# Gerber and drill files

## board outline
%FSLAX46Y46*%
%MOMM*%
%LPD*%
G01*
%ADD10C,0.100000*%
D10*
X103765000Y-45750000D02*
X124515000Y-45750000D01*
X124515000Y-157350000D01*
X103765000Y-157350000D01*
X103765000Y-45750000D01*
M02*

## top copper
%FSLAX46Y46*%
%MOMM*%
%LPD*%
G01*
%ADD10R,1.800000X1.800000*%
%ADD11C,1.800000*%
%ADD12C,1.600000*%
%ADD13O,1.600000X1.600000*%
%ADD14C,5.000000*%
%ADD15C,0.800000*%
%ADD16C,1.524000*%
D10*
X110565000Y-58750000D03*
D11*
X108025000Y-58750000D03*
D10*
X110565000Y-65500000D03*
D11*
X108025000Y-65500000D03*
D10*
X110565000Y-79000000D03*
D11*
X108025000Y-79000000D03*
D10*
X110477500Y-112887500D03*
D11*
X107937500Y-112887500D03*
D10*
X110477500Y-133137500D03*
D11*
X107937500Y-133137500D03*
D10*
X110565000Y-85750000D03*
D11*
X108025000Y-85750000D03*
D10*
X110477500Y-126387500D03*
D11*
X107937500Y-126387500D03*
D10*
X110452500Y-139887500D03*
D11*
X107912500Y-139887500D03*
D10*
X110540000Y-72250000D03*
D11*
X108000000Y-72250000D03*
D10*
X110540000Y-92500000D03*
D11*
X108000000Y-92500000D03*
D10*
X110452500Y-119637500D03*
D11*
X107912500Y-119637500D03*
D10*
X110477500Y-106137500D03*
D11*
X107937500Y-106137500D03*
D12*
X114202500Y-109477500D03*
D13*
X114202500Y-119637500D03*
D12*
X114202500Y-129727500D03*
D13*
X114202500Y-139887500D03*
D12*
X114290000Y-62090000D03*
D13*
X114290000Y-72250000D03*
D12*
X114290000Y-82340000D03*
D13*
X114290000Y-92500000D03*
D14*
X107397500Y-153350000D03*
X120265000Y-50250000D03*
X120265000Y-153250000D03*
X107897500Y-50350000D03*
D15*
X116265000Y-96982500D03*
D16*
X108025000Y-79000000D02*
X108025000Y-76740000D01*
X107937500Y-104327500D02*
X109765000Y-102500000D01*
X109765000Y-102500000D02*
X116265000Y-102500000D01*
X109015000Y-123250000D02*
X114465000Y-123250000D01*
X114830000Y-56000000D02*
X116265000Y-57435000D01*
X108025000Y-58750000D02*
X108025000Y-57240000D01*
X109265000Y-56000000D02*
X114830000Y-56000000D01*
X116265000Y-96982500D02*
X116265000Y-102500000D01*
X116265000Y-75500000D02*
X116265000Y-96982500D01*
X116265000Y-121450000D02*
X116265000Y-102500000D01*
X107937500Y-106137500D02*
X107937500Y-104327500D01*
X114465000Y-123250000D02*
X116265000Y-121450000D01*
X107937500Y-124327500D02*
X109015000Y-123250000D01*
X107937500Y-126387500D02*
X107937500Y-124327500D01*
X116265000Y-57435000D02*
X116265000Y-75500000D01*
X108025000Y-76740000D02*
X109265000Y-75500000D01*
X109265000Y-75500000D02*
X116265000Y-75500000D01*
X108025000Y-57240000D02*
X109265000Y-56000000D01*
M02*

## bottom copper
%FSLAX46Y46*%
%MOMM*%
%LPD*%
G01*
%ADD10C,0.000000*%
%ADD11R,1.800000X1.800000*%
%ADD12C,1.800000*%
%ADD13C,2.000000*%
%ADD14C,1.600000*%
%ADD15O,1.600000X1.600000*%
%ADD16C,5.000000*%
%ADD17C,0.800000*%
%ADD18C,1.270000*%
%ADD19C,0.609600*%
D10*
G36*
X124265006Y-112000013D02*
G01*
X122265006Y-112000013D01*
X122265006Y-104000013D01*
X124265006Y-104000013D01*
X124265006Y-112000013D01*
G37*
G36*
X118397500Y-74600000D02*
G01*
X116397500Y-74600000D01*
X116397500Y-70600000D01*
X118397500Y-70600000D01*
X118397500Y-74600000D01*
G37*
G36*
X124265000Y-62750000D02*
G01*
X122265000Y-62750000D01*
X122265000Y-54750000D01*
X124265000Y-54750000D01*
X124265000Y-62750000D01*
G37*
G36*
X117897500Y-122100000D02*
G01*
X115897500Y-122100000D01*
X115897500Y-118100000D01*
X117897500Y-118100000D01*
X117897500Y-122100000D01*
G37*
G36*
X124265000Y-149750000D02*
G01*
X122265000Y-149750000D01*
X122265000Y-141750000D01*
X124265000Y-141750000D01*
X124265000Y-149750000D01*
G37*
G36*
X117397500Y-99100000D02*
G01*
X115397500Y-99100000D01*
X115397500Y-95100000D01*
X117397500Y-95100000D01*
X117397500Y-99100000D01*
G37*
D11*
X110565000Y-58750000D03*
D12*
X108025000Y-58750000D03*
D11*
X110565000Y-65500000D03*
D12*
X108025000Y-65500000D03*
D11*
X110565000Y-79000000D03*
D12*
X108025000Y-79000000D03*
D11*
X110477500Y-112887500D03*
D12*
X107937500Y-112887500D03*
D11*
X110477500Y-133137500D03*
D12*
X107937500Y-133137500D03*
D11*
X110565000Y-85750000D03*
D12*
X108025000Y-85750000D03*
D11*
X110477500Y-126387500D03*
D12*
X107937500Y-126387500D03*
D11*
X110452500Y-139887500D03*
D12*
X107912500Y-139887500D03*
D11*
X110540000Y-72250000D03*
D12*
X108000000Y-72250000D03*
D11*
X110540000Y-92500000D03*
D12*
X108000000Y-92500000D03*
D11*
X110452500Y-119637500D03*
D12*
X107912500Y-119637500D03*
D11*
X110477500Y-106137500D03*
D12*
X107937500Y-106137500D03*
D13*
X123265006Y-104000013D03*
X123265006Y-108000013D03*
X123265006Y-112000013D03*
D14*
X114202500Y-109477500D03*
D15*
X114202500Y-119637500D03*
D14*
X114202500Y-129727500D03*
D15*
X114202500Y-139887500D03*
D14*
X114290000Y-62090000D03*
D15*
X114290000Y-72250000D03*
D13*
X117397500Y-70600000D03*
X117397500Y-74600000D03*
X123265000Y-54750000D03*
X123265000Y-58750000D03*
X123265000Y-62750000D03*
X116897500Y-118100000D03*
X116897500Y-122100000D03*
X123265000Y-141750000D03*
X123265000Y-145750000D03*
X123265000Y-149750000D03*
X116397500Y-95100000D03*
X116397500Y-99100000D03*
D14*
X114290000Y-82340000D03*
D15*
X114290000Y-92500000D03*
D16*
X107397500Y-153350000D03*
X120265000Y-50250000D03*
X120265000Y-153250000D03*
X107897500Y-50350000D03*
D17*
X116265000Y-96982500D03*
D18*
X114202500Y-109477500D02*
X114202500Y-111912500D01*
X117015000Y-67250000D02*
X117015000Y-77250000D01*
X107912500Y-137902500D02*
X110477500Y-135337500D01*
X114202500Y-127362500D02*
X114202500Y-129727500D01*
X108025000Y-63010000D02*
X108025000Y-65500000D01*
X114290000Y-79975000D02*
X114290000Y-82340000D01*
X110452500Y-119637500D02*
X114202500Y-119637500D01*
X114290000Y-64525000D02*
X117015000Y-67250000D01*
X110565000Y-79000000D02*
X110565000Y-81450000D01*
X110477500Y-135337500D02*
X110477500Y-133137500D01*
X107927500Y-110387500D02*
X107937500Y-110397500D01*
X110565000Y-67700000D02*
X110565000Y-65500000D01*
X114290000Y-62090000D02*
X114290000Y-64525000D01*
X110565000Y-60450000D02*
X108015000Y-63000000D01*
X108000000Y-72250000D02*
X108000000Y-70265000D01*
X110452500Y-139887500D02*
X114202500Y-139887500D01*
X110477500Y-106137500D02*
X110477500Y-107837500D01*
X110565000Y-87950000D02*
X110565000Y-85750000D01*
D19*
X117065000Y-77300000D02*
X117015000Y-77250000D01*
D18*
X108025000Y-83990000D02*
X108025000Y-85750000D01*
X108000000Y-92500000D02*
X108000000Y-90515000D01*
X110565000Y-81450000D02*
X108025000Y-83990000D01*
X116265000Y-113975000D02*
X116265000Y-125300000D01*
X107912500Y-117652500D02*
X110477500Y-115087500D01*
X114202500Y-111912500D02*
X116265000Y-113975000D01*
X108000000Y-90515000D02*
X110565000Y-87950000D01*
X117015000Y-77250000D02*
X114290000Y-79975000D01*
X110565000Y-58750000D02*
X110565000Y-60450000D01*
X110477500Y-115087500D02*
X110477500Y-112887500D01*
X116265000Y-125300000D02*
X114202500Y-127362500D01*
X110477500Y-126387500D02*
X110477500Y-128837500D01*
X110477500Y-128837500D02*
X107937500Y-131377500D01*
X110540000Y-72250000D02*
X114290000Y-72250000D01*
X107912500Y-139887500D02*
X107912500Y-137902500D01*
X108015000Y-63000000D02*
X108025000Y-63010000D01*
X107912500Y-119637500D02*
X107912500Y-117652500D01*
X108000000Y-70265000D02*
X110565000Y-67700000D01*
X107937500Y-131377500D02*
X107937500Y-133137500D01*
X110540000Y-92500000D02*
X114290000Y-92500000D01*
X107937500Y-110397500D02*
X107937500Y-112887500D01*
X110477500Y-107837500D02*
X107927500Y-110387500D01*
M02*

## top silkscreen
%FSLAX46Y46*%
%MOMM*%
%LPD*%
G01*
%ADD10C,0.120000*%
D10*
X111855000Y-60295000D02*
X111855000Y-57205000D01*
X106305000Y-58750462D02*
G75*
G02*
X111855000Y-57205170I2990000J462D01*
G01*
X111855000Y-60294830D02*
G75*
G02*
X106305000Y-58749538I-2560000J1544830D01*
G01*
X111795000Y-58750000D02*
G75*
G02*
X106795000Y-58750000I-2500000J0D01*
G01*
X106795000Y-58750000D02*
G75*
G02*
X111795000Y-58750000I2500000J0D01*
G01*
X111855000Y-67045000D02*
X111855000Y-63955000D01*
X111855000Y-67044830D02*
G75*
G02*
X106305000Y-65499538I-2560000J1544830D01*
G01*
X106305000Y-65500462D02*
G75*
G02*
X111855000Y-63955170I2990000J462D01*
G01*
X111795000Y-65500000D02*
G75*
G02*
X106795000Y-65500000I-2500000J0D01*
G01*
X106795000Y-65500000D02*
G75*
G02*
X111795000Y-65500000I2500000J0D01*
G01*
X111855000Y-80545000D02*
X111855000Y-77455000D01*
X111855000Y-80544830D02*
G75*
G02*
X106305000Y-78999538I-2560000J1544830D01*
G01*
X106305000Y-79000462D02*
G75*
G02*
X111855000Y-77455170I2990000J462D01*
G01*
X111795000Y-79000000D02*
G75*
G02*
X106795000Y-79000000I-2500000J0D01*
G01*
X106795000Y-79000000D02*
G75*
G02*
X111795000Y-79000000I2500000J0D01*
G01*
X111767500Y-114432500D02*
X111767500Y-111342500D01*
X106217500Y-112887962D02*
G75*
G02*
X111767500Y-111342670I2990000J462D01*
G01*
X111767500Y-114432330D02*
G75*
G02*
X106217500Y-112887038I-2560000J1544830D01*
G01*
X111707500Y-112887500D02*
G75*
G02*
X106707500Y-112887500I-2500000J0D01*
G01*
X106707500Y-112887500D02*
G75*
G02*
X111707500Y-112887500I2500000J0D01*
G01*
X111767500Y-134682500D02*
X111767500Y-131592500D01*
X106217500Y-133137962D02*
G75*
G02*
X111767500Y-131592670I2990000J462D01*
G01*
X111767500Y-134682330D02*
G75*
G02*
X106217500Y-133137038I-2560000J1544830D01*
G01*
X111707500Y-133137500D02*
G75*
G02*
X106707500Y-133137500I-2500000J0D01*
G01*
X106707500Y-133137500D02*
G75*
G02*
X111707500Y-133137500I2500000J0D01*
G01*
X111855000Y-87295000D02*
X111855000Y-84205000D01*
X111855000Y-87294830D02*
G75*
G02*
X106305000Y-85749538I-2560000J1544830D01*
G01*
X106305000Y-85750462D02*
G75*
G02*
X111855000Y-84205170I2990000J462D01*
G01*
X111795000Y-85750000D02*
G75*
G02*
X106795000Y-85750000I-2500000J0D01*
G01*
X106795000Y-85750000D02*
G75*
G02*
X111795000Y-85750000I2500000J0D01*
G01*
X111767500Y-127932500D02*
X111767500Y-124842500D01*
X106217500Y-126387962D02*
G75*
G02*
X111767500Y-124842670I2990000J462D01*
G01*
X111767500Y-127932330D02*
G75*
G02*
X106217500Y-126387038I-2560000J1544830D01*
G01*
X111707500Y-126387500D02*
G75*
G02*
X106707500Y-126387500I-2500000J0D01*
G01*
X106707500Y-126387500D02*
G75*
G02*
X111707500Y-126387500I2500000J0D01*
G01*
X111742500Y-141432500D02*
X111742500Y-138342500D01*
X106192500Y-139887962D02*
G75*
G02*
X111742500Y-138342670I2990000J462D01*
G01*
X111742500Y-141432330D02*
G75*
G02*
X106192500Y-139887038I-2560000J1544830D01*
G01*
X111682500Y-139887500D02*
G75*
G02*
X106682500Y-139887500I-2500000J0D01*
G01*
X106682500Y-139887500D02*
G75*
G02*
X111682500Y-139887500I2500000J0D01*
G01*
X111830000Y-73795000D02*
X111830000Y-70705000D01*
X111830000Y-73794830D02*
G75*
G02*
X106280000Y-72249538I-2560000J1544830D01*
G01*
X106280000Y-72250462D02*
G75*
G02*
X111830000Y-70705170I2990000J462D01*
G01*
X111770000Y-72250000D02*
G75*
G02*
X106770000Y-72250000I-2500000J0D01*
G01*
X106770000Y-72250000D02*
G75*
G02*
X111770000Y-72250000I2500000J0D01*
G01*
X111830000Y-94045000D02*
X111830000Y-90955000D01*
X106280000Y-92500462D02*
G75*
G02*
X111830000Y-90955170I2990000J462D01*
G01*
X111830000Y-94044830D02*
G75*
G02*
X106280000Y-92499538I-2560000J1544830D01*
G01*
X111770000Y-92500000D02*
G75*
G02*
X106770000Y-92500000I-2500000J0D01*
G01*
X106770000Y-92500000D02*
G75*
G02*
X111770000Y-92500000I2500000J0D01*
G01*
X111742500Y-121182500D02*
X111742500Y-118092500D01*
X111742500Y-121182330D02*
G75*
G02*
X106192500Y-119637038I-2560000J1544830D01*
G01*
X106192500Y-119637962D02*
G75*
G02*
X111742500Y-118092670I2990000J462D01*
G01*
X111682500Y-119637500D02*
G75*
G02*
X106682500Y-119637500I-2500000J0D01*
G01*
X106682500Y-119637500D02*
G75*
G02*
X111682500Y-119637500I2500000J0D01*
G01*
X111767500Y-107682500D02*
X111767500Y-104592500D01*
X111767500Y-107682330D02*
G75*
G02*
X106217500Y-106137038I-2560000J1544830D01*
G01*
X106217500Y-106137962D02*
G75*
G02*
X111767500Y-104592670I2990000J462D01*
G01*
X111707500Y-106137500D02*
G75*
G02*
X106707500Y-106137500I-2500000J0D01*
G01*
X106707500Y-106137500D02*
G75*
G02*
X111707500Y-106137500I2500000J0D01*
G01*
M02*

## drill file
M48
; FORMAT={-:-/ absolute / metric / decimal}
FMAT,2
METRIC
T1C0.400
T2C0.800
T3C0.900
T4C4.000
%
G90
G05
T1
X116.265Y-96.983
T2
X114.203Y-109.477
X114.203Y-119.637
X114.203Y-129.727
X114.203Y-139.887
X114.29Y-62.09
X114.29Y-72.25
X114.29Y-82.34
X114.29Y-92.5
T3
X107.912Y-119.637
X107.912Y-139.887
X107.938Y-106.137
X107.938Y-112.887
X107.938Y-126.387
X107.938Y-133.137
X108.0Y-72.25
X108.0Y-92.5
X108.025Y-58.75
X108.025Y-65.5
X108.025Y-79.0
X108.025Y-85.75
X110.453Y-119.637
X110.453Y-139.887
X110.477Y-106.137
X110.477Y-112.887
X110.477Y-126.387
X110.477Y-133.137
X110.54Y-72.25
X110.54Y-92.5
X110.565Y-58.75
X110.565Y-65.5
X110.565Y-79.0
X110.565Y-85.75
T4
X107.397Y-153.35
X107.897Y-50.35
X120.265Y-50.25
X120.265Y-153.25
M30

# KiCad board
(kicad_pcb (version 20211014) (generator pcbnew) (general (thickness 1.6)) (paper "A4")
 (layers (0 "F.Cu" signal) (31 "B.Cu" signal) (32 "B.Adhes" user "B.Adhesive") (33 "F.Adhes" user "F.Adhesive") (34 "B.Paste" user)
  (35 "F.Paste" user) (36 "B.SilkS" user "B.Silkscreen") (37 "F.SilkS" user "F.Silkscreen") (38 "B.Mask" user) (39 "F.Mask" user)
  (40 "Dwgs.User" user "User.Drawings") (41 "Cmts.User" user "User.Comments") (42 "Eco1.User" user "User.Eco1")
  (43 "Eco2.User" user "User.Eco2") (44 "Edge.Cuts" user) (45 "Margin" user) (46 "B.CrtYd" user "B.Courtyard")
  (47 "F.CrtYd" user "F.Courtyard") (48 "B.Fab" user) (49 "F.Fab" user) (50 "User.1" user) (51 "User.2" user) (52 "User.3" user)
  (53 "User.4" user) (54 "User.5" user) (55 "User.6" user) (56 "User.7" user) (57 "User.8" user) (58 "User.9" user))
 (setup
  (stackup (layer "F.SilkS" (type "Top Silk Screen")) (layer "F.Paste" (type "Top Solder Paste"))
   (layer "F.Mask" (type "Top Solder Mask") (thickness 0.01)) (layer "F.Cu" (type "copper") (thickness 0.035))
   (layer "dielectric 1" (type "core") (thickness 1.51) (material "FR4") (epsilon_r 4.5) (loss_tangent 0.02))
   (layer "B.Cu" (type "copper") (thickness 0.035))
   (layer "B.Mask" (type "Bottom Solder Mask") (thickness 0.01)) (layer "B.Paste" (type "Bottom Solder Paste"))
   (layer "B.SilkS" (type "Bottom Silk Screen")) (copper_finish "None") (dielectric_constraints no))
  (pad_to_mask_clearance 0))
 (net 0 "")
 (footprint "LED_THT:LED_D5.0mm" (layer "F.Cu") (at 110.565 58.75 180)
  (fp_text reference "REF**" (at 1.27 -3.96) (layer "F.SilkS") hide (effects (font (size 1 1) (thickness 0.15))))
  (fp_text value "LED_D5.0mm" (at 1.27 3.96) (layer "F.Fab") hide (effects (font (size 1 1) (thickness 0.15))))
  (fp_line (start -1.29 -1.545) (end -1.29 1.545) (layer "F.SilkS") (width 0.12))
  (fp_arc (start 4.26 -0.000462) (mid 2.072002 2.880433) (end -1.29 1.54483) (layer "F.SilkS") (width 0.12))
  (fp_arc (start -1.29 -1.54483) (mid 2.072002 -2.880433) (end 4.26 0.000462) (layer "F.SilkS") (width 0.12))
  (fp_circle (center 1.27 0) (end 3.77 0) (layer "F.SilkS") (width 0.12) (fill none))
  (pad "1" thru_hole rect (at 0 0 180) (size 1.8 1.8) (drill 0.9) (layers *.Cu *.Mask))
  (pad "2" thru_hole circle (at 2.54 0 180) (size 1.8 1.8) (drill 0.9) (layers *.Cu *.Mask)))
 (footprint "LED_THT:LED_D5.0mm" (layer "F.Cu") (at 110.565 65.5 180)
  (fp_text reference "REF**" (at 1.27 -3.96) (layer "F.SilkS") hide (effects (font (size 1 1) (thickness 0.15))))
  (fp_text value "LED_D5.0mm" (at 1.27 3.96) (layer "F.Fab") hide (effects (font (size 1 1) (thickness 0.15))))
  (fp_line (start -1.29 -1.545) (end -1.29 1.545) (layer "F.SilkS") (width 0.12))
  (fp_arc (start -1.29 -1.54483) (mid 2.072002 -2.880433) (end 4.26 0.000462) (layer "F.SilkS") (width 0.12))
  (fp_arc (start 4.26 -0.000462) (mid 2.072002 2.880433) (end -1.29 1.54483) (layer "F.SilkS") (width 0.12))
  (fp_circle (center 1.27 0) (end 3.77 0) (layer "F.SilkS") (width 0.12) (fill none))
  (pad "1" thru_hole rect (at 0 0 180) (size 1.8 1.8) (drill 0.9) (layers *.Cu *.Mask))
  (pad "2" thru_hole circle (at 2.54 0 180) (size 1.8 1.8) (drill 0.9) (layers *.Cu *.Mask)))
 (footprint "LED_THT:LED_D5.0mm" (layer "F.Cu") (at 110.565 79 180)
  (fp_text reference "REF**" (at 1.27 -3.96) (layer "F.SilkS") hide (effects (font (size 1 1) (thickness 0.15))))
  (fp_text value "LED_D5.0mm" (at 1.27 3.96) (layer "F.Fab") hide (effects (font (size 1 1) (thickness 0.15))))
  (fp_line (start -1.29 -1.545) (end -1.29 1.545) (layer "F.SilkS") (width 0.12))
  (fp_arc (start -1.29 -1.54483) (mid 2.072002 -2.880433) (end 4.26 0.000462) (layer "F.SilkS") (width 0.12))
  (fp_arc (start 4.26 -0.000462) (mid 2.072002 2.880433) (end -1.29 1.54483) (layer "F.SilkS") (width 0.12))
  (fp_circle (center 1.27 0) (end 3.77 0) (layer "F.SilkS") (width 0.12) (fill none))
  (pad "1" thru_hole rect (at 0 0 180) (size 1.8 1.8) (drill 0.9) (layers *.Cu *.Mask))
  (pad "2" thru_hole circle (at 2.54 0 180) (size 1.8 1.8) (drill 0.9) (layers *.Cu *.Mask)))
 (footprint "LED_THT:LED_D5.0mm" (layer "F.Cu") (at 110.4775 112.8875 180)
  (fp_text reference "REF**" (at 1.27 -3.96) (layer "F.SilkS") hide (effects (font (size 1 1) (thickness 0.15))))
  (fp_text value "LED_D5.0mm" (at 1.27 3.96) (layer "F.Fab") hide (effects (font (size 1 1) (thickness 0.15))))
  (fp_line (start -1.29 -1.545) (end -1.29 1.545) (layer "F.SilkS") (width 0.12))
  (fp_arc (start 4.26 -0.000462) (mid 2.072002 2.880433) (end -1.29 1.54483) (layer "F.SilkS") (width 0.12))
  (fp_arc (start -1.29 -1.54483) (mid 2.072002 -2.880433) (end 4.26 0.000462) (layer "F.SilkS") (width 0.12))
  (fp_circle (center 1.27 0) (end 3.77 0) (layer "F.SilkS") (width 0.12) (fill none))
  (pad "1" thru_hole rect (at 0 0 180) (size 1.8 1.8) (drill 0.9) (layers *.Cu *.Mask))
  (pad "2" thru_hole circle (at 2.54 0 180) (size 1.8 1.8) (drill 0.9) (layers *.Cu *.Mask)))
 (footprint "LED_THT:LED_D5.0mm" (layer "F.Cu") (at 110.4775 133.1375 180)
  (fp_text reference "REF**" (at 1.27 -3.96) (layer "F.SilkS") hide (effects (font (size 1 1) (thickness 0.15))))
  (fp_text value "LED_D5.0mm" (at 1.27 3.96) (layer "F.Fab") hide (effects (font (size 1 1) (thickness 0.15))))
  (fp_line (start -1.29 -1.545) (end -1.29 1.545) (layer "F.SilkS") (width 0.12))
  (fp_arc (start 4.26 -0.000462) (mid 2.072002 2.880433) (end -1.29 1.54483) (layer "F.SilkS") (width 0.12))
  (fp_arc (start -1.29 -1.54483) (mid 2.072002 -2.880433) (end 4.26 0.000462) (layer "F.SilkS") (width 0.12))
  (fp_circle (center 1.27 0) (end 3.77 0) (layer "F.SilkS") (width 0.12) (fill none))
  (pad "1" thru_hole rect (at 0 0 180) (size 1.8 1.8) (drill 0.9) (layers *.Cu *.Mask))
  (pad "2" thru_hole circle (at 2.54 0 180) (size 1.8 1.8) (drill 0.9) (layers *.Cu *.Mask)))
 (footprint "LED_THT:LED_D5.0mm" (layer "F.Cu") (at 110.565 85.75 180)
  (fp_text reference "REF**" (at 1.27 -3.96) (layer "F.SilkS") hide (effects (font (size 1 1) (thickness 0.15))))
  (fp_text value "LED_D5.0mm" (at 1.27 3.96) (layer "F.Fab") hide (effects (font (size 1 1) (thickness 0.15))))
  (fp_line (start -1.29 -1.545) (end -1.29 1.545) (layer "F.SilkS") (width 0.12))
  (fp_arc (start -1.29 -1.54483) (mid 2.072002 -2.880433) (end 4.26 0.000462) (layer "F.SilkS") (width 0.12))
  (fp_arc (start 4.26 -0.000462) (mid 2.072002 2.880433) (end -1.29 1.54483) (layer "F.SilkS") (width 0.12))
  (fp_circle (center 1.27 0) (end 3.77 0) (layer "F.SilkS") (width 0.12) (fill none))
  (pad "1" thru_hole rect (at 0 0 180) (size 1.8 1.8) (drill 0.9) (layers *.Cu *.Mask))
  (pad "2" thru_hole circle (at 2.54 0 180) (size 1.8 1.8) (drill 0.9) (layers *.Cu *.Mask)))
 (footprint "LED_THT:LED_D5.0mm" (layer "F.Cu") (at 110.4775 126.3875 180)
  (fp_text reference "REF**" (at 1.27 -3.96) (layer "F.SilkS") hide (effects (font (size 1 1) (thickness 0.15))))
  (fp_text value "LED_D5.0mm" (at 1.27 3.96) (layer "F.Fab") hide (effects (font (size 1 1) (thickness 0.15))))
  (fp_line (start -1.29 -1.545) (end -1.29 1.545) (layer "F.SilkS") (width 0.12))
  (fp_arc (start 4.26 -0.000462) (mid 2.072002 2.880433) (end -1.29 1.54483) (layer "F.SilkS") (width 0.12))
  (fp_arc (start -1.29 -1.54483) (mid 2.072002 -2.880433) (end 4.26 0.000462) (layer "F.SilkS") (width 0.12))
  (fp_circle (center 1.27 0) (end 3.77 0) (layer "F.SilkS") (width 0.12) (fill none))
  (pad "1" thru_hole rect (at 0 0 180) (size 1.8 1.8) (drill 0.9) (layers *.Cu *.Mask))
  (pad "2" thru_hole circle (at 2.54 0 180) (size 1.8 1.8) (drill 0.9) (layers *.Cu *.Mask)))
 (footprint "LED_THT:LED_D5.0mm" (layer "F.Cu") (at 110.4525 139.8875 180)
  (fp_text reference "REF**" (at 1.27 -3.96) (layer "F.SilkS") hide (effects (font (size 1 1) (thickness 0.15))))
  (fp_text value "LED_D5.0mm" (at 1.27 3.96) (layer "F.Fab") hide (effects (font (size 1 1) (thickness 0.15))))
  (fp_line (start -1.29 -1.545) (end -1.29 1.545) (layer "F.SilkS") (width 0.12))
  (fp_arc (start 4.26 -0.000462) (mid 2.072002 2.880433) (end -1.29 1.54483) (layer "F.SilkS") (width 0.12))
  (fp_arc (start -1.29 -1.54483) (mid 2.072002 -2.880433) (end 4.26 0.000462) (layer "F.SilkS") (width 0.12))
  (fp_circle (center 1.27 0) (end 3.77 0) (layer "F.SilkS") (width 0.12) (fill none))
  (pad "1" thru_hole rect (at 0 0 180) (size 1.8 1.8) (drill 0.9) (layers *.Cu *.Mask))
  (pad "2" thru_hole circle (at 2.54 0 180) (size 1.8 1.8) (drill 0.9) (layers *.Cu *.Mask)))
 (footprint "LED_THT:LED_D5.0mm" (layer "F.Cu") (at 110.54 72.25 180)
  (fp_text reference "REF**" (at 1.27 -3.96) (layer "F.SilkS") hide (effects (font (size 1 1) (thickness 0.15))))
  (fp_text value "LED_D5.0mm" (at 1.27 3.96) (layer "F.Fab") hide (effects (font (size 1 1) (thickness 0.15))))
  (fp_line (start -1.29 -1.545) (end -1.29 1.545) (layer "F.SilkS") (width 0.12))
  (fp_arc (start -1.29 -1.54483) (mid 2.072002 -2.880433) (end 4.26 0.000462) (layer "F.SilkS") (width 0.12))
  (fp_arc (start 4.26 -0.000462) (mid 2.072002 2.880433) (end -1.29 1.54483) (layer "F.SilkS") (width 0.12))
  (fp_circle (center 1.27 0) (end 3.77 0) (layer "F.SilkS") (width 0.12) (fill none))
  (pad "1" thru_hole rect (at 0 0 180) (size 1.8 1.8) (drill 0.9) (layers *.Cu *.Mask))
  (pad "2" thru_hole circle (at 2.54 0 180) (size 1.8 1.8) (drill 0.9) (layers *.Cu *.Mask)))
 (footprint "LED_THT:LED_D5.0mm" (layer "F.Cu") (at 110.54 92.5 180)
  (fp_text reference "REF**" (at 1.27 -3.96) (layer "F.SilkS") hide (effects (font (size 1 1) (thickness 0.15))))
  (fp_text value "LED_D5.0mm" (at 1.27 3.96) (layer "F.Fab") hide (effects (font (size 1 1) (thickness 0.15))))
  (fp_line (start -1.29 -1.545) (end -1.29 1.545) (layer "F.SilkS") (width 0.12))
  (fp_arc (start 4.26 -0.000462) (mid 2.072002 2.880433) (end -1.29 1.54483) (layer "F.SilkS") (width 0.12))
  (fp_arc (start -1.29 -1.54483) (mid 2.072002 -2.880433) (end 4.26 0.000462) (layer "F.SilkS") (width 0.12))
  (fp_circle (center 1.27 0) (end 3.77 0) (layer "F.SilkS") (width 0.12) (fill none))
  (pad "1" thru_hole rect (at 0 0 180) (size 1.8 1.8) (drill 0.9) (layers *.Cu *.Mask))
  (pad "2" thru_hole circle (at 2.54 0 180) (size 1.8 1.8) (drill 0.9) (layers *.Cu *.Mask)))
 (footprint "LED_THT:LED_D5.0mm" (layer "F.Cu") (at 110.4525 119.6375 180)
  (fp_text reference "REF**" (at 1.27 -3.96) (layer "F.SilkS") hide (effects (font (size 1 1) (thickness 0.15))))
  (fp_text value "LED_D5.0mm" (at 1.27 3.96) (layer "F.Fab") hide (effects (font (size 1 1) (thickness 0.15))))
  (fp_line (start -1.29 -1.545) (end -1.29 1.545) (layer "F.SilkS") (width 0.12))
  (fp_arc (start -1.29 -1.54483) (mid 2.072002 -2.880433) (end 4.26 0.000462) (layer "F.SilkS") (width 0.12))
  (fp_arc (start 4.26 -0.000462) (mid 2.072002 2.880433) (end -1.29 1.54483) (layer "F.SilkS") (width 0.12))
  (fp_circle (center 1.27 0) (end 3.77 0) (layer "F.SilkS") (width 0.12) (fill none))
  (pad "1" thru_hole rect (at 0 0 180) (size 1.8 1.8) (drill 0.9) (layers *.Cu *.Mask))
  (pad "2" thru_hole circle (at 2.54 0 180) (size 1.8 1.8) (drill 0.9) (layers *.Cu *.Mask)))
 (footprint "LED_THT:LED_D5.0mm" (layer "F.Cu") (at 110.4775 106.1375 180)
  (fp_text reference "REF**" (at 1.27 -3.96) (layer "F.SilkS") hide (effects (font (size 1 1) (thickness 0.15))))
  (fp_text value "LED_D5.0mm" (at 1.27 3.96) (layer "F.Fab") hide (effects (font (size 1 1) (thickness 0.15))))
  (fp_line (start -1.29 -1.545) (end -1.29 1.545) (layer "F.SilkS") (width 0.12))
  (fp_arc (start -1.29 -1.54483) (mid 2.072002 -2.880433) (end 4.26 0.000462) (layer "F.SilkS") (width 0.12))
  (fp_arc (start 4.26 -0.000462) (mid 2.072002 2.880433) (end -1.29 1.54483) (layer "F.SilkS") (width 0.12))
  (fp_circle (center 1.27 0) (end 3.77 0) (layer "F.SilkS") (width 0.12) (fill none))
  (pad "1" thru_hole rect (at 0 0 180) (size 1.8 1.8) (drill 0.9) (layers *.Cu *.Mask))
  (pad "2" thru_hole circle (at 2.54 0 180) (size 1.8 1.8) (drill 0.9) (layers *.Cu *.Mask)))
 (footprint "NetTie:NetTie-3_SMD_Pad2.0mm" (layer "B.Cu") (at 123.265006 108.000013 -90)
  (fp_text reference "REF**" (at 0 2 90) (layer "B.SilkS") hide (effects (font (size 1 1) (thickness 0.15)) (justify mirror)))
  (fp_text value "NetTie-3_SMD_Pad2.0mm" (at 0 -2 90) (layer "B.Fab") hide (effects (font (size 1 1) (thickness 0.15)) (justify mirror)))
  (fp_poly (pts (xy -4 1) (xy 4 1) (xy 4 -1) (xy -4 -1)) (layer "B.Cu") (width 0) (fill solid))
  (pad "1" smd circle (at -4 0 270) (size 2 2) (layers "B.Cu")) (pad "2" smd circle (at 0 0 270) (size 2 2) (layers "B.Cu"))
  (pad "3" smd circle (at 4 0 270) (size 2 2) (layers "B.Cu")))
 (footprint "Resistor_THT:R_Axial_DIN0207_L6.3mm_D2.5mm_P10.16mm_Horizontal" (layer "B.Cu") (at 114.2025 109.4775 -90)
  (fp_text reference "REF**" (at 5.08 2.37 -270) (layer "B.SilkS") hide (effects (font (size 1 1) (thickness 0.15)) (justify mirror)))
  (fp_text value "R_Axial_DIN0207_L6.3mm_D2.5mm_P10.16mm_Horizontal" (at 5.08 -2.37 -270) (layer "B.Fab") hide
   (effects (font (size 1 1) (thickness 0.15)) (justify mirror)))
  (pad "1" thru_hole circle (at 0 0 270) (size 1.6 1.6) (drill 0.8) (layers *.Cu *.Mask))
  (pad "2" thru_hole oval (at 10.16 0 270) (size 1.6 1.6) (drill 0.8) (layers *.Cu *.Mask)))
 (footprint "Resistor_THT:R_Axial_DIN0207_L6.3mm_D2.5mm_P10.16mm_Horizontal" (layer "B.Cu") (at 114.2025 129.7275 -90)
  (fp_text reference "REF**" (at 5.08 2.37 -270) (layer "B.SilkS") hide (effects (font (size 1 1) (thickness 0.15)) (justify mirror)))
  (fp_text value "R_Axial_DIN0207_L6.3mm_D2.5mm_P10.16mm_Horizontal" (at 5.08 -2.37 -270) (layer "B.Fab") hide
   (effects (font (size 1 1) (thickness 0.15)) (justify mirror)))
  (pad "1" thru_hole circle (at 0 0 270) (size 1.6 1.6) (drill 0.8) (layers *.Cu *.Mask))
  (pad "2" thru_hole oval (at 10.16 0 270) (size 1.6 1.6) (drill 0.8) (layers *.Cu *.Mask)))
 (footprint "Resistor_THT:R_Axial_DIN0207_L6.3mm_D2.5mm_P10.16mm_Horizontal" (layer "B.Cu") (at 114.29 62.09 -90)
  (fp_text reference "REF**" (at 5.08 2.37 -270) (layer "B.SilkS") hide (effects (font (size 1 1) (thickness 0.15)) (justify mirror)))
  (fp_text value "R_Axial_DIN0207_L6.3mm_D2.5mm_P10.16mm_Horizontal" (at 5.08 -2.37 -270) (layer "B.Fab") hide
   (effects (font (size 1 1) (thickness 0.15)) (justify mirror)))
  (pad "1" thru_hole circle (at 0 0 270) (size 1.6 1.6) (drill 0.8) (layers *.Cu *.Mask))
  (pad "2" thru_hole oval (at 10.16 0 270) (size 1.6 1.6) (drill 0.8) (layers *.Cu *.Mask)))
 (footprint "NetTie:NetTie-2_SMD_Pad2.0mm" (layer "B.Cu") (at 117.3975 72.6 -90)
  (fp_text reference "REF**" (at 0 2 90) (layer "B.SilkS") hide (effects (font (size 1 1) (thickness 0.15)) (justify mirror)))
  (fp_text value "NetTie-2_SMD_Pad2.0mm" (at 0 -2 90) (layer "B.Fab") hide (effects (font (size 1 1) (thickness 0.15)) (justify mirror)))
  (fp_poly (pts (xy -2 1) (xy 2 1) (xy 2 -1) (xy -2 -1)) (layer "B.Cu") (width 0) (fill solid))
  (pad "1" smd circle (at -2 0 270) (size 2 2) (layers "B.Cu")) (pad "2" smd circle (at 2 0 270) (size 2 2) (layers "B.Cu")))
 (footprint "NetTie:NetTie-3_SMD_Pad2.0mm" (layer "B.Cu") (at 123.265 58.75 -90)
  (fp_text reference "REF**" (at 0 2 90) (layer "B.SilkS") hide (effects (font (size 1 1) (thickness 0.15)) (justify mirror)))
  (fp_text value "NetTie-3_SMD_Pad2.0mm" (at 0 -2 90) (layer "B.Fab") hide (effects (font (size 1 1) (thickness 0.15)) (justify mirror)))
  (fp_poly (pts (xy -4 1) (xy 4 1) (xy 4 -1) (xy -4 -1)) (layer "B.Cu") (width 0) (fill solid))
  (pad "1" smd circle (at -4 0 270) (size 2 2) (layers "B.Cu")) (pad "2" smd circle (at 0 0 270) (size 2 2) (layers "B.Cu"))
  (pad "3" smd circle (at 4 0 270) (size 2 2) (layers "B.Cu")))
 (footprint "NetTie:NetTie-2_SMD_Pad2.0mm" (layer "B.Cu") (at 116.8975 120.1 -90)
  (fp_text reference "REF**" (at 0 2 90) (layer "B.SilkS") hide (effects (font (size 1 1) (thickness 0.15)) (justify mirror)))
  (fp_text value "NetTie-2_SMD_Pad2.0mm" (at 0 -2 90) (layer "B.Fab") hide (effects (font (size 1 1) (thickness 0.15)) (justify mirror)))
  (fp_poly (pts (xy -2 1) (xy 2 1) (xy 2 -1) (xy -2 -1)) (layer "B.Cu") (width 0) (fill solid))
  (pad "1" smd circle (at -2 0 270) (size 2 2) (layers "B.Cu")) (pad "2" smd circle (at 2 0 270) (size 2 2) (layers "B.Cu")))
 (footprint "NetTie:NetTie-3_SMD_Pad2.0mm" (layer "B.Cu") (at 123.265 145.75 -90)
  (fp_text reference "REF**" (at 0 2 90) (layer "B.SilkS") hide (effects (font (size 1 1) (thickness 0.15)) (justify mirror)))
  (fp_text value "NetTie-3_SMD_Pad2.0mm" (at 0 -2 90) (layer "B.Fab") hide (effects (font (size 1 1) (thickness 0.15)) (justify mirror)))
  (fp_poly (pts (xy -4 1) (xy 4 1) (xy 4 -1) (xy -4 -1)) (layer "B.Cu") (width 0) (fill solid))
  (pad "1" smd circle (at -4 0 270) (size 2 2) (layers "B.Cu")) (pad "2" smd circle (at 0 0 270) (size 2 2) (layers "B.Cu"))
  (pad "3" smd circle (at 4 0 270) (size 2 2) (layers "B.Cu")))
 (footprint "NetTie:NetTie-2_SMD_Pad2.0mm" (layer "B.Cu") (at 116.3975 97.1 -90)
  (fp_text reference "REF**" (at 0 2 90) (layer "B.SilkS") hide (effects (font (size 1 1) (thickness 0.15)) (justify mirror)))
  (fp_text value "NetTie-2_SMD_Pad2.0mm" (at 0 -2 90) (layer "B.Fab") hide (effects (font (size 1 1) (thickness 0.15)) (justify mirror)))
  (fp_poly (pts (xy -2 1) (xy 2 1) (xy 2 -1) (xy -2 -1)) (layer "B.Cu") (width 0) (fill solid))
  (pad "1" smd circle (at -2 0 270) (size 2 2) (layers "B.Cu")) (pad "2" smd circle (at 2 0 270) (size 2 2) (layers "B.Cu")))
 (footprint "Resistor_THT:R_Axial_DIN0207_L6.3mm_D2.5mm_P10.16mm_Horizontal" (layer "B.Cu") (at 114.29 82.34 -90)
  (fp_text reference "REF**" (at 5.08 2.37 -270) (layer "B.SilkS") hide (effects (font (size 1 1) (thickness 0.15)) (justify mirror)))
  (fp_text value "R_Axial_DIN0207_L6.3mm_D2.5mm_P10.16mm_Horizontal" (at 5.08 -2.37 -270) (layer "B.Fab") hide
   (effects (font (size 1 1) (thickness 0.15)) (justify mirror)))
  (pad "1" thru_hole circle (at 0 0 270) (size 1.6 1.6) (drill 0.8) (layers *.Cu *.Mask))
  (pad "2" thru_hole oval (at 10.16 0 270) (size 1.6 1.6) (drill 0.8) (layers *.Cu *.Mask)))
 (gr_rect (start 124.515 157.35) (end 103.765 45.75) (layer "Edge.Cuts") (width 0.1) (fill none))
 (segment (start 108.025 79) (end 108.025 76.74) (width 1.524) (layer "F.Cu") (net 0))
 (segment (start 107.9375 104.3275) (end 109.765 102.5) (width 1.524) (layer "F.Cu") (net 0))
 (segment (start 109.765 102.5) (end 116.265 102.5) (width 1.524) (layer "F.Cu") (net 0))
 (segment (start 109.015 123.25) (end 114.465 123.25) (width 1.524) (layer "F.Cu") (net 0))
 (segment (start 114.83 56) (end 116.265 57.435) (width 1.524) (layer "F.Cu") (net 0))
 (segment (start 108.025 58.75) (end 108.025 57.24) (width 1.524) (layer "F.Cu") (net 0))
 (segment (start 109.265 56) (end 114.83 56) (width 1.524) (layer "F.Cu") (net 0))
 (segment (start 116.265 96.9825) (end 116.265 102.5) (width 1.524) (layer "F.Cu") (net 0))
 (segment (start 116.265 75.5) (end 116.265 96.9825) (width 1.524) (layer "F.Cu") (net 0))
 (segment (start 116.265 121.45) (end 116.265 102.5) (width 1.524) (layer "F.Cu") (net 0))
 (segment (start 107.9375 106.1375) (end 107.9375 104.3275) (width 1.524) (layer "F.Cu") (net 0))
 (segment (start 114.465 123.25) (end 116.265 121.45) (width 1.524) (layer "F.Cu") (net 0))
 (segment (start 107.9375 124.3275) (end 109.015 123.25) (width 1.524) (layer "F.Cu") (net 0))
 (segment (start 107.9375 126.3875) (end 107.9375 124.3275) (width 1.524) (layer "F.Cu") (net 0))
 (segment (start 116.265 57.435) (end 116.265 75.5) (width 1.524) (layer "F.Cu") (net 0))
 (segment (start 108.025 76.74) (end 109.265 75.5) (width 1.524) (layer "F.Cu") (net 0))
 (segment (start 109.265 75.5) (end 116.265 75.5) (width 1.524) (layer "F.Cu") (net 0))
 (segment (start 108.025 57.24) (end 109.265 56) (width 1.524) (layer "F.Cu") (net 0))
 (via (at 107.3975 153.35) (size 5) (drill 4) (layers "F.Cu" "B.Cu") (free) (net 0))
 (via (at 120.265 50.25) (size 5) (drill 4) (layers "F.Cu" "B.Cu") (free) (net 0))
 (via (at 120.265 153.25) (size 5) (drill 4) (layers "F.Cu" "B.Cu") (free) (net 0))
 (via (at 107.8975 50.35) (size 5) (drill 4) (layers "F.Cu" "B.Cu") (free) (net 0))
 (via (at 116.265 96.9825) (size 0.8) (drill 0.4) (layers "F.Cu" "B.Cu") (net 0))
 (segment (start 114.2025 109.4775) (end 114.2025 111.9125) (width 1.27) (layer "B.Cu") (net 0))
 (segment (start 117.015 67.25) (end 117.015 77.25) (width 1.27) (layer "B.Cu") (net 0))
 (segment (start 107.9125 137.9025) (end 110.4775 135.3375) (width 1.27) (layer "B.Cu") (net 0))
 (segment (start 114.2025 127.3625) (end 114.2025 129.7275) (width 1.27) (layer "B.Cu") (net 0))
 (segment (start 108.025 63.01) (end 108.025 65.5) (width 1.27) (layer "B.Cu") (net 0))
 (segment (start 114.29 79.975) (end 114.29 82.34) (width 1.27) (layer "B.Cu") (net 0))
 (segment (start 110.4525 119.6375) (end 114.2025 119.6375) (width 1.27) (layer "B.Cu") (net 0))
 (segment (start 114.29 64.525) (end 117.015 67.25) (width 1.27) (layer "B.Cu") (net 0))
 (segment (start 110.565 79) (end 110.565 81.45) (width 1.27) (layer "B.Cu") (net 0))
 (segment (start 110.4775 135.3375) (end 110.4775 133.1375) (width 1.27) (layer "B.Cu") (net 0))
 (segment (start 107.9275 110.3875) (end 107.9375 110.3975) (width 1.27) (layer "B.Cu") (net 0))
 (segment (start 110.565 67.7) (end 110.565 65.5) (width 1.27) (layer "B.Cu") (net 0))
 (segment (start 114.29 62.09) (end 114.29 64.525) (width 1.27) (layer "B.Cu") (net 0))
 (segment (start 110.565 60.45) (end 108.015 63) (width 1.27) (layer "B.Cu") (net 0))
 (segment (start 108 72.25) (end 108 70.265) (width 1.27) (layer "B.Cu") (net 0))
 (segment (start 110.4525 139.8875) (end 114.2025 139.8875) (width 1.27) (layer "B.Cu") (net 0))
 (segment (start 110.4775 106.1375) (end 110.4775 107.8375) (width 1.27) (layer "B.Cu") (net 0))
 (segment (start 110.565 87.95) (end 110.565 85.75) (width 1.27) (layer "B.Cu") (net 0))
 (segment (start 117.065 77.3) (end 117.015 77.25) (width 0.6096) (layer "B.Cu") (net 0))
 (segment (start 108.025 83.99) (end 108.025 85.75) (width 1.27) (layer "B.Cu") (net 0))
 (segment (start 108 92.5) (end 108 90.515) (width 1.27) (layer "B.Cu") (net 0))
 (segment (start 110.565 81.45) (end 108.025 83.99) (width 1.27) (layer "B.Cu") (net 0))
 (segment (start 116.265 113.975) (end 116.265 125.3) (width 1.27) (layer "B.Cu") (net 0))
 (segment (start 107.9125 117.6525) (end 110.4775 115.0875) (width 1.27) (layer "B.Cu") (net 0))
 (segment (start 114.2025 111.9125) (end 116.265 113.975) (width 1.27) (layer "B.Cu") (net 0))
 (segment (start 108 90.515) (end 110.565 87.95) (width 1.27) (layer "B.Cu") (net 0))
 (segment (start 117.015 77.25) (end 114.29 79.975) (width 1.27) (layer "B.Cu") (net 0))
 (segment (start 110.565 58.75) (end 110.565 60.45) (width 1.27) (layer "B.Cu") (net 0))
 (segment (start 110.4775 115.0875) (end 110.4775 112.8875) (width 1.27) (layer "B.Cu") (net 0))
 (segment (start 116.265 125.3) (end 114.2025 127.3625) (width 1.27) (layer "B.Cu") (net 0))
 (segment (start 110.4775 126.3875) (end 110.4775 128.8375) (width 1.27) (layer "B.Cu") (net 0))
 (segment (start 110.4775 128.8375) (end 107.9375 131.3775) (width 1.27) (layer "B.Cu") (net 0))
 (segment (start 110.54 72.25) (end 114.29 72.25) (width 1.27) (layer "B.Cu") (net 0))
 (segment (start 107.9125 139.8875) (end 107.9125 137.9025) (width 1.27) (layer "B.Cu") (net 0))
 (segment (start 108.015 63) (end 108.025 63.01) (width 1.27) (layer "B.Cu") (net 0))
 (segment (start 107.9125 119.6375) (end 107.9125 117.6525) (width 1.27) (layer "B.Cu") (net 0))
 (segment (start 108 70.265) (end 110.565 67.7) (width 1.27) (layer "B.Cu") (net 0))
 (segment (start 107.9375 131.3775) (end 107.9375 133.1375) (width 1.27) (layer "B.Cu") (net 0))
 (segment (start 110.54 92.5) (end 114.29 92.5) (width 1.27) (layer "B.Cu") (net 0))
 (segment (start 107.9375 110.3975) (end 107.9375 112.8875) (width 1.27) (layer "B.Cu") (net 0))
 (segment (start 110.4775 107.8375) (end 107.9275 110.3875) (width 1.27) (layer "B.Cu") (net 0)))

